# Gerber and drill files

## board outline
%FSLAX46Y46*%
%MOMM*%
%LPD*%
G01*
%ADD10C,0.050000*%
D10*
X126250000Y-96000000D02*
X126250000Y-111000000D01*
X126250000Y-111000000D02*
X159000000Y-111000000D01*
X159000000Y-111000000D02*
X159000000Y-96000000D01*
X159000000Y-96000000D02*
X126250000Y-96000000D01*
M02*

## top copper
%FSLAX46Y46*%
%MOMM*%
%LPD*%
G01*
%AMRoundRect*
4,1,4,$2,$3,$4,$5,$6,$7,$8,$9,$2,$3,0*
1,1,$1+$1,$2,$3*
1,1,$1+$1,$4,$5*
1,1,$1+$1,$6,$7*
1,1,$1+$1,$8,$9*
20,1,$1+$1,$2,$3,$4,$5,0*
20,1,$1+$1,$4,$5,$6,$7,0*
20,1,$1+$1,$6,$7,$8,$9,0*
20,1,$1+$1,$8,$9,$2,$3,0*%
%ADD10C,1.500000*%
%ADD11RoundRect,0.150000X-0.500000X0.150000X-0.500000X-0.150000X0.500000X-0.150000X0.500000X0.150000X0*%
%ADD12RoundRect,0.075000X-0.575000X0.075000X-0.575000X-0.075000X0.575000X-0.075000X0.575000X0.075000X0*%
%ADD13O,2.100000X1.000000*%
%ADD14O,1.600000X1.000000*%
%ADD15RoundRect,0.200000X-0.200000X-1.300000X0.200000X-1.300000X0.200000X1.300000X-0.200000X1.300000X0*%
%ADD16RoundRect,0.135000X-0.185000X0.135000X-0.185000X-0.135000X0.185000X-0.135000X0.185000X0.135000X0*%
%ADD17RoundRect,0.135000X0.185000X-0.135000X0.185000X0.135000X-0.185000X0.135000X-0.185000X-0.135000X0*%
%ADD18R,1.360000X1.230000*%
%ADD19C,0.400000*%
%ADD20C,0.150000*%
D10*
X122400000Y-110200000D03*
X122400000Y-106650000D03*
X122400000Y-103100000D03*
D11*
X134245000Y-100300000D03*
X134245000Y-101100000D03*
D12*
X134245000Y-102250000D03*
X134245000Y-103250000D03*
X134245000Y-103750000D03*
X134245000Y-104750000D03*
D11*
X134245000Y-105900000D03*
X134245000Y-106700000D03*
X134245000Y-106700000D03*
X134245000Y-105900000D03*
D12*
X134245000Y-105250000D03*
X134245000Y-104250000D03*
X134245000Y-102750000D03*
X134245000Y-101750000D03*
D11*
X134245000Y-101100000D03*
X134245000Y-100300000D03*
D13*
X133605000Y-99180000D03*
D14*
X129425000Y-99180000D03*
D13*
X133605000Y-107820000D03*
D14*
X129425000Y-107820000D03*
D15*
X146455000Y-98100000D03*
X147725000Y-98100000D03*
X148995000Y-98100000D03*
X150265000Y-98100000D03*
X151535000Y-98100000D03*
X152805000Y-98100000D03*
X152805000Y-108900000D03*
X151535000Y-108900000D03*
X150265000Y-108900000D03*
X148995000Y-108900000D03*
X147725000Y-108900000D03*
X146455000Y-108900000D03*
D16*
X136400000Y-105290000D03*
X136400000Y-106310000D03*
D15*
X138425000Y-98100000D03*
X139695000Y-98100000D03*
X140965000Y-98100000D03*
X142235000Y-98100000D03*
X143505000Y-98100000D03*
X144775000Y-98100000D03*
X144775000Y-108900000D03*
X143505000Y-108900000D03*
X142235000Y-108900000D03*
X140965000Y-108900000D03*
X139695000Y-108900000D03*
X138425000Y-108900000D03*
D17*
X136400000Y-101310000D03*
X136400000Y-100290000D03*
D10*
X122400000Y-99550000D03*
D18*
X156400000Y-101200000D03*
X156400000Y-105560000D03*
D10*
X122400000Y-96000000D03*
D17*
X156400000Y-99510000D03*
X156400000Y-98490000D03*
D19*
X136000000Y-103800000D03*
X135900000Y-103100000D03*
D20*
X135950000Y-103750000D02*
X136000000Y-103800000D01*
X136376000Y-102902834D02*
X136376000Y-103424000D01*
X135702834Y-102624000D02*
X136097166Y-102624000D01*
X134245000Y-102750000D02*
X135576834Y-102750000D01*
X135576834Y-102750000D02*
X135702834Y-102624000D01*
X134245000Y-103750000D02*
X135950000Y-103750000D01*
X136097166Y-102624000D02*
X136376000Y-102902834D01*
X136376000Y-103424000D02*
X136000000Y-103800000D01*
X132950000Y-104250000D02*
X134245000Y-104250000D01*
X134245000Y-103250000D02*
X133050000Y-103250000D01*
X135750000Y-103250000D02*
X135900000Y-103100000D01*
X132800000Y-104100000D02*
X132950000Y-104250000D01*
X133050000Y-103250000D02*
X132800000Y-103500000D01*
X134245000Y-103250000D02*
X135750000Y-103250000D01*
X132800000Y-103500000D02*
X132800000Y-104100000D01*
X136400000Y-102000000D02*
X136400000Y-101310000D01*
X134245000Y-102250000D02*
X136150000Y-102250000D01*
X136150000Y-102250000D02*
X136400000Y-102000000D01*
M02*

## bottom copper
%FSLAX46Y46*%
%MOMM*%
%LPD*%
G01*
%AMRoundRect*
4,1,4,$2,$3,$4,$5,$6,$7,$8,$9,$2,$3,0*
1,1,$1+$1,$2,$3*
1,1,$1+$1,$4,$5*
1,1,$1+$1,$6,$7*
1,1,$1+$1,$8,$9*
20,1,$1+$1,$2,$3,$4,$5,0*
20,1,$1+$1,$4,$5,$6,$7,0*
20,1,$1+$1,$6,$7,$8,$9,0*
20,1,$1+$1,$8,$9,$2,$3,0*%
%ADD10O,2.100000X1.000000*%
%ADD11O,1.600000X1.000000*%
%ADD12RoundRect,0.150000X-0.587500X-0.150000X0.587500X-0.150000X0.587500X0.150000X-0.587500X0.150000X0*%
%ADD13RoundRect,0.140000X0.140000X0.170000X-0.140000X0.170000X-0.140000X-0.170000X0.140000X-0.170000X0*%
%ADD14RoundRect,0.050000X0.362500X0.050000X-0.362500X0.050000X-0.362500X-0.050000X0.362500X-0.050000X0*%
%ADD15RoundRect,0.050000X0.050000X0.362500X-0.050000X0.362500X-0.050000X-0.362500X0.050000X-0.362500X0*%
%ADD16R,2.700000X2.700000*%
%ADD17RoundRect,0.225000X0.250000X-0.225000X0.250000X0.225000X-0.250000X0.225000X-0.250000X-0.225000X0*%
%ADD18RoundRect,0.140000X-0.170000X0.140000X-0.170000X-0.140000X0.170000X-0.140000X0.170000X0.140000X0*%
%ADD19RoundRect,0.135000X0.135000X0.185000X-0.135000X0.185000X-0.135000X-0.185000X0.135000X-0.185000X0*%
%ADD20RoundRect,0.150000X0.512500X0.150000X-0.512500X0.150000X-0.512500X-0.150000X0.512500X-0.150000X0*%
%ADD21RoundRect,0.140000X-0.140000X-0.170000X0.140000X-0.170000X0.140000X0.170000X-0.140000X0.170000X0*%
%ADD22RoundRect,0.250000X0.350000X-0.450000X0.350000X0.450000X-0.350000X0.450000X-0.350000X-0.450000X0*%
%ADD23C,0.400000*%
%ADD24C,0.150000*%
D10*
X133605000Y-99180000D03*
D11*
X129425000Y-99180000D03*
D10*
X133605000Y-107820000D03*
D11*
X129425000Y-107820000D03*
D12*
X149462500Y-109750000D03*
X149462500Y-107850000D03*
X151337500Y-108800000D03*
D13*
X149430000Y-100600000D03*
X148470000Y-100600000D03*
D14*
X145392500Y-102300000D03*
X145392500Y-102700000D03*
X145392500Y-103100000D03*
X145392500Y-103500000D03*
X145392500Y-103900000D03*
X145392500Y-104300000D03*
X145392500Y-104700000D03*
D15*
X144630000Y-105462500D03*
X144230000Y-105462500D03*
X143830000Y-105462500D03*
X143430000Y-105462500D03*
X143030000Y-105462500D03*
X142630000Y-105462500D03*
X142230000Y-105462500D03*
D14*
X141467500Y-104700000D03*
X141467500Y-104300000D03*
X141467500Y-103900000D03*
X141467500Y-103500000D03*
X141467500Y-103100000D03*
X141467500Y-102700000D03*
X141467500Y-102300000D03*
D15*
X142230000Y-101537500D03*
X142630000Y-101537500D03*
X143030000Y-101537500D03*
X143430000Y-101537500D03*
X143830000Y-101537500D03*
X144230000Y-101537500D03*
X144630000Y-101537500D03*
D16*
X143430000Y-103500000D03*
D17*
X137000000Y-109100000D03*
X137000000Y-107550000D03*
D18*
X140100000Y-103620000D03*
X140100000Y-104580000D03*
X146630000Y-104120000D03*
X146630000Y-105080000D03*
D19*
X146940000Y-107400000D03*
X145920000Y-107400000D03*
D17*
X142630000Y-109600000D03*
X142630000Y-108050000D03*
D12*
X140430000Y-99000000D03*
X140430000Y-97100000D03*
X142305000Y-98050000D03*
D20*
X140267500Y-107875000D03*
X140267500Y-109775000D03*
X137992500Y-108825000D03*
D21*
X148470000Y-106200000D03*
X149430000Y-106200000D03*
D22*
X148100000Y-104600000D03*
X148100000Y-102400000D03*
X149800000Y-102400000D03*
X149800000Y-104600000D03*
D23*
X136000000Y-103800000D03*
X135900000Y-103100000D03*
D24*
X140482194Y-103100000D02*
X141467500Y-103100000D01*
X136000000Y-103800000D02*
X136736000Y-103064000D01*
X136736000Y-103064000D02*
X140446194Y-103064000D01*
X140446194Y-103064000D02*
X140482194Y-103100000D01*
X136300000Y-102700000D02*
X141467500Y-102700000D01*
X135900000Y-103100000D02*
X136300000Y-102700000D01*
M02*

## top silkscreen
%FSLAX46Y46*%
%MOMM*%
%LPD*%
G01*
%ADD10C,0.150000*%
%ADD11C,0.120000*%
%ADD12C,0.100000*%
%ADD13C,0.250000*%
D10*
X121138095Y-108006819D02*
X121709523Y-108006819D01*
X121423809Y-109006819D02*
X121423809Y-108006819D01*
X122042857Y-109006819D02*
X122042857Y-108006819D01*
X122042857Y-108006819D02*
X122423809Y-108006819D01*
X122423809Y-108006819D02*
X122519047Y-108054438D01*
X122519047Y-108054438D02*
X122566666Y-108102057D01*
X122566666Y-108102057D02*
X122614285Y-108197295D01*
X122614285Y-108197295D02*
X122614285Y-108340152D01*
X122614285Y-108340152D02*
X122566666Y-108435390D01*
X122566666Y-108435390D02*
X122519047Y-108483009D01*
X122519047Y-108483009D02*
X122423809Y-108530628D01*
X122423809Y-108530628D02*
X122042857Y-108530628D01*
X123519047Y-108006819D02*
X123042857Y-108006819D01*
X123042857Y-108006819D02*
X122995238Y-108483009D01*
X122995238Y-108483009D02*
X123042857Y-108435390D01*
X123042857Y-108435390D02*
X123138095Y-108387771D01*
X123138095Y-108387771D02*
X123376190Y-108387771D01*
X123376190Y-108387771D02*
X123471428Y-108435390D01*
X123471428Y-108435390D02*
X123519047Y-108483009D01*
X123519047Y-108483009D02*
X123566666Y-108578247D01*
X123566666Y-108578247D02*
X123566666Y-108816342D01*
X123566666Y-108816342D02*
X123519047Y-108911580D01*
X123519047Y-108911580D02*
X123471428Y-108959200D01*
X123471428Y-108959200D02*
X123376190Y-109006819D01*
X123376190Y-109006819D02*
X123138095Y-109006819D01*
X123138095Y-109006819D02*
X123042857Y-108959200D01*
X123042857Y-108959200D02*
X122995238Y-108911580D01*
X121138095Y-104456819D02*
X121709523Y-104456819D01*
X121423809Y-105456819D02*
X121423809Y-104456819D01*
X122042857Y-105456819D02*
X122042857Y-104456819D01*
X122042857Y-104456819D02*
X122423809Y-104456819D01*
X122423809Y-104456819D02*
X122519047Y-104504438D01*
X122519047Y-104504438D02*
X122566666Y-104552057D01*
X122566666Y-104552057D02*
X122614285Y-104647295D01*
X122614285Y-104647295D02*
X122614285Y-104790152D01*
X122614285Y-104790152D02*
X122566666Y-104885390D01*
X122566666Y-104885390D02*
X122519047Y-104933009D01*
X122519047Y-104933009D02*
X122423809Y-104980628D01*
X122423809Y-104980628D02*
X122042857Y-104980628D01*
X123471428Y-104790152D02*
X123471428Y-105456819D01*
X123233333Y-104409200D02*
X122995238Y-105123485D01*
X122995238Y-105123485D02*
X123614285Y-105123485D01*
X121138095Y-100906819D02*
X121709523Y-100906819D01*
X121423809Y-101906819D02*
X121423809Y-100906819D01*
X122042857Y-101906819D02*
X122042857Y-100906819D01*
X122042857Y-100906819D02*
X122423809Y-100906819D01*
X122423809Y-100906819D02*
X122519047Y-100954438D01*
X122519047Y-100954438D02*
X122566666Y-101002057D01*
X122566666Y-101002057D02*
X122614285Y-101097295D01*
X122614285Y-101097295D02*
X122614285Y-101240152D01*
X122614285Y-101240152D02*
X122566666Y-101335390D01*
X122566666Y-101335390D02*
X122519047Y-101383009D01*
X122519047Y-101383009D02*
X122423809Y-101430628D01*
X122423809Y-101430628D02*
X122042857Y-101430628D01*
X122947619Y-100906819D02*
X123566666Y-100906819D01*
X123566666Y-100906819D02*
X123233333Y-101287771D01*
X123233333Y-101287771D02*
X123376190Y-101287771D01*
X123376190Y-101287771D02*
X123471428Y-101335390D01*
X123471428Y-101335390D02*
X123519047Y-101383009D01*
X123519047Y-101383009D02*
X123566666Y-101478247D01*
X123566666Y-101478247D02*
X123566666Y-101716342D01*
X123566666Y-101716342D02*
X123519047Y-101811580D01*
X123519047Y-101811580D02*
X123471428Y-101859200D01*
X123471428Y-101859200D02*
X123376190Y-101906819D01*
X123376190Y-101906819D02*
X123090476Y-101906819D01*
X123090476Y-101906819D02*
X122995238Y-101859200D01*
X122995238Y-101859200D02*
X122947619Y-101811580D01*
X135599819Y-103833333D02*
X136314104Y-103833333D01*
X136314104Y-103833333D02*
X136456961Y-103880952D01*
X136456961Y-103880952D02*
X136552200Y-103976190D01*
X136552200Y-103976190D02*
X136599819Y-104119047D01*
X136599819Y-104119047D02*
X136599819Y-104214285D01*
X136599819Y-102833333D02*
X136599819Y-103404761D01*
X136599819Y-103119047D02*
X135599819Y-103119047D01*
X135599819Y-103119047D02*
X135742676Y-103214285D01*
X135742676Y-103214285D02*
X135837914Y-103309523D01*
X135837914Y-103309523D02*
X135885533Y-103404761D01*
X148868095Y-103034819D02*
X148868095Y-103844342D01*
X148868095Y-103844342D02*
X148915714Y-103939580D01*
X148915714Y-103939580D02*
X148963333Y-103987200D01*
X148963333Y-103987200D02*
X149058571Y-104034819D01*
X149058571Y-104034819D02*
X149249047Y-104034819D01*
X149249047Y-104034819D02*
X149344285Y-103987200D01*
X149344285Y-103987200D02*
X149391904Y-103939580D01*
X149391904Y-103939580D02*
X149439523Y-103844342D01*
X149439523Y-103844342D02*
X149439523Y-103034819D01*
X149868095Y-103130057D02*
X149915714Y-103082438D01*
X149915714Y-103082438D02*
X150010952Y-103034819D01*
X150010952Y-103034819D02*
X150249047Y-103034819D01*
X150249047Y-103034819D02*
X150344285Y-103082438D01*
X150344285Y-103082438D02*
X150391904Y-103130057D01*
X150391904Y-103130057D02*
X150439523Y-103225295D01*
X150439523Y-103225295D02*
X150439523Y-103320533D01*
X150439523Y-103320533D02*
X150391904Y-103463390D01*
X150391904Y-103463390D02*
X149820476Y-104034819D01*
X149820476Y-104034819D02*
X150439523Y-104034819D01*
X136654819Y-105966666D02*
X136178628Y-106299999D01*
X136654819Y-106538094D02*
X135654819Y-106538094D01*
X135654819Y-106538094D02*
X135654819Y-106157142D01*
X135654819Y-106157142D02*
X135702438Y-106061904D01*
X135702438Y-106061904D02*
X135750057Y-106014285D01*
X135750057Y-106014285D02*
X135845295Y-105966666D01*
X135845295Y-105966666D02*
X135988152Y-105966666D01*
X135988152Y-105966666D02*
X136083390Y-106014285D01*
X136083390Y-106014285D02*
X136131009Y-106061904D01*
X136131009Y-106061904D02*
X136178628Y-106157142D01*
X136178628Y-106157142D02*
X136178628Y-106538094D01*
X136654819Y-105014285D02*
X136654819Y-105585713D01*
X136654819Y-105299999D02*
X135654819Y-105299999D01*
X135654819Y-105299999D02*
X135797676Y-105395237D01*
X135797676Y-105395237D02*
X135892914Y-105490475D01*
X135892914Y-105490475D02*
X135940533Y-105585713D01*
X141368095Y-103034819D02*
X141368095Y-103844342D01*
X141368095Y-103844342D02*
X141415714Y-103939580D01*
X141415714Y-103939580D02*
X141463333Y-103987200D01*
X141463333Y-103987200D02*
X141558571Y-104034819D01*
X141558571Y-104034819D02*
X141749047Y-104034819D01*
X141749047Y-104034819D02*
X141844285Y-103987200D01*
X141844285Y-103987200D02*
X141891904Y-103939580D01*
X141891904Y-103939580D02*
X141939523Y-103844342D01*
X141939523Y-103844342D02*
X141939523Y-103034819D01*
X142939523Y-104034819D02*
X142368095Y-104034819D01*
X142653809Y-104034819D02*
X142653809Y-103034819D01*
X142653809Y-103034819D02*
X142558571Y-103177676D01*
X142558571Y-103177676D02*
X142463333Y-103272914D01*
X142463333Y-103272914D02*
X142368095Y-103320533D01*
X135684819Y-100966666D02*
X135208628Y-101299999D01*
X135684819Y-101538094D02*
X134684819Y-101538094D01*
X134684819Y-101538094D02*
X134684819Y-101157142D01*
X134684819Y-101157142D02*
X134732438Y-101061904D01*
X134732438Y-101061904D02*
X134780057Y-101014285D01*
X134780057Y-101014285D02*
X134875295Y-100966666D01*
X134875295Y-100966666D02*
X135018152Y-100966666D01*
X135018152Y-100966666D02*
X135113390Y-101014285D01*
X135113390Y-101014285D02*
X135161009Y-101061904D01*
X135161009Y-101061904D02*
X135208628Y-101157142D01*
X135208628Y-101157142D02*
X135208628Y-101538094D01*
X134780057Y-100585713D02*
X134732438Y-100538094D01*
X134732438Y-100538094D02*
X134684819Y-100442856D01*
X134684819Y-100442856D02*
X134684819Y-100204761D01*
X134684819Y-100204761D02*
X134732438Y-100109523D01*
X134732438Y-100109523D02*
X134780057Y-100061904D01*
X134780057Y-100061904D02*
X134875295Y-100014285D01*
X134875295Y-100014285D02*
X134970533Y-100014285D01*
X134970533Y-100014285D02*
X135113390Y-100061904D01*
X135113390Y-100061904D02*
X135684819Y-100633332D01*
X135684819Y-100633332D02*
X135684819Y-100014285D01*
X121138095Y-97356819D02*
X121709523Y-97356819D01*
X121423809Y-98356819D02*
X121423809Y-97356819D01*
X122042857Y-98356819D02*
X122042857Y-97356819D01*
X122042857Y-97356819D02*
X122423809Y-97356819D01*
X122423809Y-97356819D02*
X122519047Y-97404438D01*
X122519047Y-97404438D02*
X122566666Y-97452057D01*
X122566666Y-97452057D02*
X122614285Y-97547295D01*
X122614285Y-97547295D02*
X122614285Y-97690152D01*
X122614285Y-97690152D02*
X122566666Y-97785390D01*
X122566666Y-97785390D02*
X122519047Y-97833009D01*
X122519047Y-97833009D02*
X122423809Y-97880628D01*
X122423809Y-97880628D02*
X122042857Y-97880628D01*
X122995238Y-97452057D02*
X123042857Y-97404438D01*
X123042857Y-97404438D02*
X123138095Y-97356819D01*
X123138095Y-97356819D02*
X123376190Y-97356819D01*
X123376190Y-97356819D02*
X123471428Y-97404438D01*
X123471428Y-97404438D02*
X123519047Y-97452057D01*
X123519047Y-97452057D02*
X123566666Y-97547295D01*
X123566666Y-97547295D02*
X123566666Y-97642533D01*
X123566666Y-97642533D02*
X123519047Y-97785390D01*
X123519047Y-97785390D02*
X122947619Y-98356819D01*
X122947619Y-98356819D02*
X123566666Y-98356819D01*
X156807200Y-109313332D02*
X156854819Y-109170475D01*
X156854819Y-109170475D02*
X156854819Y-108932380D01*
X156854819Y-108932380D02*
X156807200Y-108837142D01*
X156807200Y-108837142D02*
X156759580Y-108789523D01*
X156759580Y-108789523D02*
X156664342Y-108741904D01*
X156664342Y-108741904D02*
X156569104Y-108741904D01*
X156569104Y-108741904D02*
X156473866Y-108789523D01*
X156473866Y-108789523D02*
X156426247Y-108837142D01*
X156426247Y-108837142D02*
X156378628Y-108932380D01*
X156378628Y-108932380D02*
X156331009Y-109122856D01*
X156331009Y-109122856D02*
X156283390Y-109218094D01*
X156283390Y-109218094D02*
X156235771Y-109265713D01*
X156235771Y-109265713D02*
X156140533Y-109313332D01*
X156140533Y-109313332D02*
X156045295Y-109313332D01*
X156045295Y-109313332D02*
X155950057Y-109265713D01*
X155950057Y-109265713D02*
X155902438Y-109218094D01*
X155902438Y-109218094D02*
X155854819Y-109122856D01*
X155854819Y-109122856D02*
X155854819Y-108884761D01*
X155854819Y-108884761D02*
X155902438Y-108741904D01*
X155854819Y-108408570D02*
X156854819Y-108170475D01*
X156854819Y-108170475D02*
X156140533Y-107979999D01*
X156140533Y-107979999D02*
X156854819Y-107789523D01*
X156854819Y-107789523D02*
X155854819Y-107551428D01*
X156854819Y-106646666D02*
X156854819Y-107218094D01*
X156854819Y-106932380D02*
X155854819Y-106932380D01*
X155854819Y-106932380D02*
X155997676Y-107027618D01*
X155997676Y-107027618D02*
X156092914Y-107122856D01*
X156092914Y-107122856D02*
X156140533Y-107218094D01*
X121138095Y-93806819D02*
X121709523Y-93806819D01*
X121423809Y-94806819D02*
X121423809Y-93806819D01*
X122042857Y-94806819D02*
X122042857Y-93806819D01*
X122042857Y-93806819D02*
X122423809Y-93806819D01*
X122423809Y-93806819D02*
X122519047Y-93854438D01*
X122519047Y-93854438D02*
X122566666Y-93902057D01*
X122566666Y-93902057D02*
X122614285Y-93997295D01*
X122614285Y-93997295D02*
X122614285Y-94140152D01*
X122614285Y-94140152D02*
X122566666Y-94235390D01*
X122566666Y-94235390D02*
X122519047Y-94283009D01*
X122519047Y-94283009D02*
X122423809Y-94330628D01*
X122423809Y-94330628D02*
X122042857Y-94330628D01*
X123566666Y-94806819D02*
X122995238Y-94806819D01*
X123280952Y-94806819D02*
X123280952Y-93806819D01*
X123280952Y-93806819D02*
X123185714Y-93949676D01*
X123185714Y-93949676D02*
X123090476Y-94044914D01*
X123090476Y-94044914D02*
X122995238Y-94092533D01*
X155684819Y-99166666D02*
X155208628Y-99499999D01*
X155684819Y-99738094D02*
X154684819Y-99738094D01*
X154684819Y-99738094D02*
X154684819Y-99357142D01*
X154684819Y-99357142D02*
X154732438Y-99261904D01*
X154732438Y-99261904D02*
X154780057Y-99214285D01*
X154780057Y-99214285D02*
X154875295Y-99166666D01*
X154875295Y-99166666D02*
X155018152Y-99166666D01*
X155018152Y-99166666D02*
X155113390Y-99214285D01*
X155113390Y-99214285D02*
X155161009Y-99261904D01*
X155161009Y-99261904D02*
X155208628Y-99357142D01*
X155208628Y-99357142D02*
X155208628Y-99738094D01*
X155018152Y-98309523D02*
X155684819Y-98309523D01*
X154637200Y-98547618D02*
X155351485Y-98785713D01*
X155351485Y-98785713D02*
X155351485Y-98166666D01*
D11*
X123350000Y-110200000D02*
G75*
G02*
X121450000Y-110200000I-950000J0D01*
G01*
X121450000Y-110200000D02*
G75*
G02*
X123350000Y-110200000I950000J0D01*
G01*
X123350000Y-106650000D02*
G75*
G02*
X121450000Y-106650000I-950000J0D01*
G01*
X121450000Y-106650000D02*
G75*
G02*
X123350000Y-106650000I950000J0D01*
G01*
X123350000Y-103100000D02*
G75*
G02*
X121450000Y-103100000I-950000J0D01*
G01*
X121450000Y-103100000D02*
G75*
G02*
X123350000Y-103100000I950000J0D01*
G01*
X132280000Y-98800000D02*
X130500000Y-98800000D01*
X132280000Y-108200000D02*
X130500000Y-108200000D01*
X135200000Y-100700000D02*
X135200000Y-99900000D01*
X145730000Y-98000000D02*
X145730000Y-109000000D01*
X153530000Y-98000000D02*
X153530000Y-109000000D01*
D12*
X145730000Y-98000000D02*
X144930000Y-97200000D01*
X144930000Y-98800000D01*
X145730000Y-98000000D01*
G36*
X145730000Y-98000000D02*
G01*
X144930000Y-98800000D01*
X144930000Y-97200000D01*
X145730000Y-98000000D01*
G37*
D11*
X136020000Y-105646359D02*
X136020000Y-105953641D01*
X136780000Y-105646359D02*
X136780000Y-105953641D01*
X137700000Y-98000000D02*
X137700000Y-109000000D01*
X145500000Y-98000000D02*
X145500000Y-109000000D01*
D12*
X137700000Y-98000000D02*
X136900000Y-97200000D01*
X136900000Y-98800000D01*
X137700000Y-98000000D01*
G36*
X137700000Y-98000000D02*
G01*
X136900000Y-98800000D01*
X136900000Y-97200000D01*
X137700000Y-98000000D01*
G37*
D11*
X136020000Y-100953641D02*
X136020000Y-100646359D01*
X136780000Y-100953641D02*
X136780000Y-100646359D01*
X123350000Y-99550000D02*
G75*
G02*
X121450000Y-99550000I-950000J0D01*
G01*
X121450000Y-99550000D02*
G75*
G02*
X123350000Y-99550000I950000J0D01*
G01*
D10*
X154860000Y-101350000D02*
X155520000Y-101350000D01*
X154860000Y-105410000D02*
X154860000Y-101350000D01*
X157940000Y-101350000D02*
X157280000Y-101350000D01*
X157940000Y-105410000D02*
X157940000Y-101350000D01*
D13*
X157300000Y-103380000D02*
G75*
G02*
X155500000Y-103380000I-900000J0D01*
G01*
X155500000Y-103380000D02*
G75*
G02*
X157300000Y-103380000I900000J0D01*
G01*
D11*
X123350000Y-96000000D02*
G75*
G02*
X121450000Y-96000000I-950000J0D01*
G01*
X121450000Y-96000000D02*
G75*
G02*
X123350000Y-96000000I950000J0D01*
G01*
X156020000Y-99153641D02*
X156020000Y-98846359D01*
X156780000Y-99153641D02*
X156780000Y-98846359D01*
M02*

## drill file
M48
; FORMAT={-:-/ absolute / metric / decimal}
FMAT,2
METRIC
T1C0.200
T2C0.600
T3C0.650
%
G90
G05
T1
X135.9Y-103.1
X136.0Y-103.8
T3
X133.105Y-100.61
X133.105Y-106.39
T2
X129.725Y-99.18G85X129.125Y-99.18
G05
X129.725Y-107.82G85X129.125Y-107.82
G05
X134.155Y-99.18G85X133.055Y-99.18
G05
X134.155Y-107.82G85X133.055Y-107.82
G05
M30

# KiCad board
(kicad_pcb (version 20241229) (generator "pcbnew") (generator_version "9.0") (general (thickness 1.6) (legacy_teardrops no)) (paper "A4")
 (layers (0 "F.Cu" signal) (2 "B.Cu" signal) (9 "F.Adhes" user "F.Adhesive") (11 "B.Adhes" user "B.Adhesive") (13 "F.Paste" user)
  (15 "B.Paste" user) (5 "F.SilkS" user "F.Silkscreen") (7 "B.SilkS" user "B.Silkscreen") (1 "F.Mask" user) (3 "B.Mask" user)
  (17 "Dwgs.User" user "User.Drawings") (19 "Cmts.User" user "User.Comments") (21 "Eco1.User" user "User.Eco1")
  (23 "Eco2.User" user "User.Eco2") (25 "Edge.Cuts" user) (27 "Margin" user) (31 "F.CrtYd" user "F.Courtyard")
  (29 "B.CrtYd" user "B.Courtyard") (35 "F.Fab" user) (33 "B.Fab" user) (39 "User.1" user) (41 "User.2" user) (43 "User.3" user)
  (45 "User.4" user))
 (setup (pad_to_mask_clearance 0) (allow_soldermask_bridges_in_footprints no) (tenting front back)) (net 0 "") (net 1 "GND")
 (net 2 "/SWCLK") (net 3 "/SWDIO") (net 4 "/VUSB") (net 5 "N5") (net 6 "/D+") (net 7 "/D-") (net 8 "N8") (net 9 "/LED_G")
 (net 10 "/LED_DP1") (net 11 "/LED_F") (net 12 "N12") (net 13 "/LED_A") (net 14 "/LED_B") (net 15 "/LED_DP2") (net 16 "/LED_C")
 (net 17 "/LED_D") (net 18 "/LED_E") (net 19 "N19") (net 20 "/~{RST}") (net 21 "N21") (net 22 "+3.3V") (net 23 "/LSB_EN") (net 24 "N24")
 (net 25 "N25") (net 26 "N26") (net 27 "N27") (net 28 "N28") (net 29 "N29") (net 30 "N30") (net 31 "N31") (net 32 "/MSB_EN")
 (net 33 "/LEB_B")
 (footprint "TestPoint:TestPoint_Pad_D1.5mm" (layer "F.Cu") (at 122.4 110.2)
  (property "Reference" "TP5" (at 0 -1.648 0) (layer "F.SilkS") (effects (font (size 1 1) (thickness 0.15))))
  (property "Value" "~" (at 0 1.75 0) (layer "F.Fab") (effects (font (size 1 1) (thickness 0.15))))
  (fp_circle (center 0 0) (end 0 0.95) (stroke (width 0.12) (type solid)) (fill no) (layer "F.SilkS"))
  (pad "1" smd circle (at 0 0) (size 1.5 1.5) (layers "F.Cu" "F.Mask") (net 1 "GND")))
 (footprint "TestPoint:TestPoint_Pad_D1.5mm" (layer "F.Cu") (at 122.4 106.65)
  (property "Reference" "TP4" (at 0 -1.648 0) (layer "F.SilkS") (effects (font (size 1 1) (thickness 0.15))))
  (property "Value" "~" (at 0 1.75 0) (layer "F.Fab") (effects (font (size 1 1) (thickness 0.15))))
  (fp_circle (center 0 0) (end 0 0.95) (stroke (width 0.12) (type solid)) (fill no) (layer "F.SilkS"))
  (pad "1" smd circle (at 0 0) (size 1.5 1.5) (layers "F.Cu" "F.Mask") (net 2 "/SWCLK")))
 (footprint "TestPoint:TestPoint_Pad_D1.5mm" (layer "F.Cu") (at 122.4 103.1)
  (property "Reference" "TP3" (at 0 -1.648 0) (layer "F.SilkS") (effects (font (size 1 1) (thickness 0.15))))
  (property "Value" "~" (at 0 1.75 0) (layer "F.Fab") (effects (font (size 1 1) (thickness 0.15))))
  (fp_circle (center 0 0) (end 0 0.95) (stroke (width 0.12) (type solid)) (fill no) (layer "F.SilkS"))
  (pad "1" smd circle (at 0 0) (size 1.5 1.5) (layers "F.Cu" "F.Mask") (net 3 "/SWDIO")))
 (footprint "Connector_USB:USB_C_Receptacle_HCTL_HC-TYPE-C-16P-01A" (layer "F.Cu") (at 130.5 103.5 -90)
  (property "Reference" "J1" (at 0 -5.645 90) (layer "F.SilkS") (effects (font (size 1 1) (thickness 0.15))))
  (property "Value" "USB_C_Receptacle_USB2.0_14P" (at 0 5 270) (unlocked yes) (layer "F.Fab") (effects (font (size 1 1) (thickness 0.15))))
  (fp_line (start -4.7 -1.78) (end -4.7 0) (stroke (width 0.12) (type solid)) (layer "F.SilkS"))
  (fp_line (start 4.7 -1.78) (end 4.7 0) (stroke (width 0.12) (type solid)) (layer "F.SilkS"))
  (fp_line (start -2.8 -4.7) (end -3.6 -4.7) (stroke (width 0.12) (type default)) (layer "F.SilkS"))
  (pad "" np_thru_hole circle (at -2.89 -2.605 270) (size 0.65 0.65) (drill 0.65) (layers "*.Mask"))
  (pad "" np_thru_hole circle (at 2.89 -2.605 270) (size 0.65 0.65) (drill 0.65) (layers "*.Mask"))
  (pad "A1" smd roundrect (at -3.2 -3.745 270) (size 0.6 1.3) (layers "F.Cu" "F.Mask" "F.Paste") (roundrect_rratio 0.25) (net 1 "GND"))
  (pad "A4" smd roundrect (at -2.4 -3.745 270) (size 0.6 1.3) (layers "F.Cu" "F.Mask" "F.Paste") (roundrect_rratio 0.25) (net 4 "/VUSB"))
  (pad "A5" smd roundrect (at -1.25 -3.745 270) (size 0.3 1.3) (layers "F.Cu" "F.Mask" "F.Paste") (roundrect_rratio 0.25) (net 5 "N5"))
  (pad "A6" smd roundrect (at -0.25 -3.745 270) (size 0.3 1.3) (layers "F.Cu" "F.Mask" "F.Paste") (roundrect_rratio 0.25) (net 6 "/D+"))
  (pad "A7" smd roundrect (at 0.25 -3.745 270) (size 0.3 1.3) (layers "F.Cu" "F.Mask" "F.Paste") (roundrect_rratio 0.25) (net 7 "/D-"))
  (pad "A8" smd roundrect (at 1.25 -3.745 270) (size 0.3 1.3) (layers "F.Cu" "F.Mask" "F.Paste") (roundrect_rratio 0.25))
  (pad "A9" smd roundrect (at 2.4 -3.745 270) (size 0.6 1.3) (layers "F.Cu" "F.Mask" "F.Paste") (roundrect_rratio 0.25) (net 4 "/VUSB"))
  (pad "A12" smd roundrect (at 3.2 -3.745 270) (size 0.6 1.3) (layers "F.Cu" "F.Mask" "F.Paste") (roundrect_rratio 0.25) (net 1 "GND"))
  (pad "B1" smd roundrect (at 3.2 -3.745 270) (size 0.6 1.3) (layers "F.Cu" "F.Mask" "F.Paste") (roundrect_rratio 0.25) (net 1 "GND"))
  (pad "B4" smd roundrect (at 2.4 -3.745 270) (size 0.6 1.3) (layers "F.Cu" "F.Mask" "F.Paste") (roundrect_rratio 0.25) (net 4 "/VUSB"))
  (pad "B5" smd roundrect (at 1.75 -3.745 270) (size 0.3 1.3) (layers "F.Cu" "F.Mask" "F.Paste") (roundrect_rratio 0.25) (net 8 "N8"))
  (pad "B6" smd roundrect (at 0.75 -3.745 270) (size 0.3 1.3) (layers "F.Cu" "F.Mask" "F.Paste") (roundrect_rratio 0.25) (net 6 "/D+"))
  (pad "B7" smd roundrect (at -0.75 -3.745 270) (size 0.3 1.3) (layers "F.Cu" "F.Mask" "F.Paste") (roundrect_rratio 0.25) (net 7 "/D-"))
  (pad "B8" smd roundrect (at -1.75 -3.745 270) (size 0.3 1.3) (layers "F.Cu" "F.Mask" "F.Paste") (roundrect_rratio 0.25))
  (pad "B9" smd roundrect (at -2.4 -3.745 270) (size 0.6 1.3) (layers "F.Cu" "F.Mask" "F.Paste") (roundrect_rratio 0.25) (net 4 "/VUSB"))
  (pad "B12" smd roundrect (at -3.2 -3.745 270) (size 0.6 1.3) (layers "F.Cu" "F.Mask" "F.Paste") (roundrect_rratio 0.25) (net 1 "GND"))
  (pad "S1" thru_hole oval (at -4.32 -3.105 270) (size 1 2.1) (drill oval 0.6 1.7) (layers "*.Cu" "*.Mask") (remove_unused_layers no)
   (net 1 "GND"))
  (pad "S1" thru_hole oval (at -4.32 1.075 270) (size 1 1.6) (drill oval 0.6 1.2) (layers "*.Cu" "*.Mask") (remove_unused_layers no)
   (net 1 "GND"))
  (pad "S1" thru_hole oval (at 4.32 -3.105 270) (size 1 2.1) (drill oval 0.6 1.7) (layers "*.Cu" "*.Mask") (remove_unused_layers no)
   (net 1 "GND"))
  (pad "S1" thru_hole oval (at 4.32 1.075 270) (size 1 1.6) (drill oval 0.6 1.2) (layers "*.Cu" "*.Mask") (remove_unused_layers no)
   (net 1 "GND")))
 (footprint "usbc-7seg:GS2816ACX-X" (layer "F.Cu") (at 149.63 103.5)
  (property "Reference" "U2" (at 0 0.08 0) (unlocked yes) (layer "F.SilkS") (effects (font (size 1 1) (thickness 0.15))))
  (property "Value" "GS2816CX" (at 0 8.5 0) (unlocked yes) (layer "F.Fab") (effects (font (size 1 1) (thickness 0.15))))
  (fp_line (start -3.9 -5.5) (end -3.9 5.5) (stroke (width 0.12) (type solid)) (layer "F.SilkS"))
  (fp_line (start 3.9 -5.5) (end 3.9 5.5) (stroke (width 0.12) (type solid)) (layer "F.SilkS"))
  (fp_poly (pts (xy -3.9 -5.5) (xy -4.7 -6.3) (xy -4.7 -4.7)) (stroke (width 0.1) (type solid)) (fill yes) (layer "F.SilkS"))
  (pad "1" smd roundrect (at -3.175 -5.4) (size 0.8 3) (layers "F.Cu" "F.Mask" "F.Paste") (roundrect_rratio 0.25) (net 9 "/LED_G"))
  (pad "2" smd roundrect (at -1.905 -5.4) (size 0.8 3) (layers "F.Cu" "F.Mask" "F.Paste") (roundrect_rratio 0.25) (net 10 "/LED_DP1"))
  (pad "3" smd roundrect (at -0.635 -5.4) (size 0.8 3) (layers "F.Cu" "F.Mask" "F.Paste") (roundrect_rratio 0.25) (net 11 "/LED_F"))
  (pad "4" smd roundrect (at 0.635 -5.4) (size 0.8 3) (layers "F.Cu" "F.Mask" "F.Paste") (roundrect_rratio 0.25) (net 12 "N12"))
  (pad "5" smd roundrect (at 1.905 -5.4) (size 0.8 3) (layers "F.Cu" "F.Mask" "F.Paste") (roundrect_rratio 0.25) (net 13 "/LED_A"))
  (pad "6" smd roundrect (at 3.175 -5.4) (size 0.8 3) (layers "F.Cu" "F.Mask" "F.Paste") (roundrect_rratio 0.25) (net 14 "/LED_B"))
  (pad "7" smd roundrect (at 3.175 5.4) (size 0.8 3) (layers "F.Cu" "F.Mask" "F.Paste") (roundrect_rratio 0.25) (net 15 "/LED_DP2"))
  (pad "8" smd roundrect (at 1.905 5.4) (size 0.8 3) (layers "F.Cu" "F.Mask" "F.Paste") (roundrect_rratio 0.25) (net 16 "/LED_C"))
  (pad "9" smd roundrect (at 0.635 5.4) (size 0.8 3) (layers "F.Cu" "F.Mask" "F.Paste") (roundrect_rratio 0.25) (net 12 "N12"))
  (pad "10" smd roundrect (at -0.635 5.4) (size 0.8 3) (layers "F.Cu" "F.Mask" "F.Paste") (roundrect_rratio 0.25) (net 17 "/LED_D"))
  (pad "11" smd roundrect (at -1.905 5.4) (size 0.8 3) (layers "F.Cu" "F.Mask" "F.Paste") (roundrect_rratio 0.25) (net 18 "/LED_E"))
  (pad "12" smd roundrect (at -3.175 5.4) (size 0.8 3) (layers "F.Cu" "F.Mask" "F.Paste") (roundrect_rratio 0.25)))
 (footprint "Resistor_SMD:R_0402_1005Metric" (layer "F.Cu") (at 136.4 105.8 -90)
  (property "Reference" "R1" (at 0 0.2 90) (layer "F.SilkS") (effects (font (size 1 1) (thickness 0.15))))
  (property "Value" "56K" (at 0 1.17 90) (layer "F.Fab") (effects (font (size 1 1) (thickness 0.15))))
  (fp_line (start -0.153641 0.38) (end 0.153641 0.38) (stroke (width 0.12) (type solid)) (layer "F.SilkS"))
  (fp_line (start -0.153641 -0.38) (end 0.153641 -0.38) (stroke (width 0.12) (type solid)) (layer "F.SilkS"))
  (pad "1" smd roundrect (at -0.51 0 270) (size 0.54 0.64) (layers "F.Cu" "F.Mask" "F.Paste") (roundrect_rratio 0.25) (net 8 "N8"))
  (pad "2" smd roundrect (at 0.51 0 270) (size 0.54 0.64) (layers "F.Cu" "F.Mask" "F.Paste") (roundrect_rratio 0.25) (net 1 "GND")))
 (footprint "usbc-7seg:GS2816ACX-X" (layer "F.Cu") (at 141.6 103.5)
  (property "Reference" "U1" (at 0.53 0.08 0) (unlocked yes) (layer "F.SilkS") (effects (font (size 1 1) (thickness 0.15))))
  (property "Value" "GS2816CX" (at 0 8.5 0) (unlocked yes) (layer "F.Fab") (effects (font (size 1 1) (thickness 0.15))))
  (fp_line (start -3.9 -5.5) (end -3.9 5.5) (stroke (width 0.12) (type solid)) (layer "F.SilkS"))
  (fp_line (start 3.9 -5.5) (end 3.9 5.5) (stroke (width 0.12) (type solid)) (layer "F.SilkS"))
  (fp_poly (pts (xy -3.9 -5.5) (xy -4.7 -6.3) (xy -4.7 -4.7)) (stroke (width 0.1) (type solid)) (fill yes) (layer "F.SilkS"))
  (pad "1" smd roundrect (at -3.175 -5.4) (size 0.8 3) (layers "F.Cu" "F.Mask" "F.Paste") (roundrect_rratio 0.25) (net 9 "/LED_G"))
  (pad "2" smd roundrect (at -1.905 -5.4) (size 0.8 3) (layers "F.Cu" "F.Mask" "F.Paste") (roundrect_rratio 0.25) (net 10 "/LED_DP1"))
  (pad "3" smd roundrect (at -0.635 -5.4) (size 0.8 3) (layers "F.Cu" "F.Mask" "F.Paste") (roundrect_rratio 0.25) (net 11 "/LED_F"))
  (pad "4" smd roundrect (at 0.635 -5.4) (size 0.8 3) (layers "F.Cu" "F.Mask" "F.Paste") (roundrect_rratio 0.25) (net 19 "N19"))
  (pad "5" smd roundrect (at 1.905 -5.4) (size 0.8 3) (layers "F.Cu" "F.Mask" "F.Paste") (roundrect_rratio 0.25) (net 13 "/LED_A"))
  (pad "6" smd roundrect (at 3.175 -5.4) (size 0.8 3) (layers "F.Cu" "F.Mask" "F.Paste") (roundrect_rratio 0.25) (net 14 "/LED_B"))
  (pad "7" smd roundrect (at 3.175 5.4) (size 0.8 3) (layers "F.Cu" "F.Mask" "F.Paste") (roundrect_rratio 0.25) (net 15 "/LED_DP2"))
  (pad "8" smd roundrect (at 1.905 5.4) (size 0.8 3) (layers "F.Cu" "F.Mask" "F.Paste") (roundrect_rratio 0.25) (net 16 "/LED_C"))
  (pad "9" smd roundrect (at 0.635 5.4) (size 0.8 3) (layers "F.Cu" "F.Mask" "F.Paste") (roundrect_rratio 0.25) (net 19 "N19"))
  (pad "10" smd roundrect (at -0.635 5.4) (size 0.8 3) (layers "F.Cu" "F.Mask" "F.Paste") (roundrect_rratio 0.25) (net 17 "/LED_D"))
  (pad "11" smd roundrect (at -1.905 5.4) (size 0.8 3) (layers "F.Cu" "F.Mask" "F.Paste") (roundrect_rratio 0.25) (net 18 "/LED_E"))
  (pad "12" smd roundrect (at -3.175 5.4) (size 0.8 3) (layers "F.Cu" "F.Mask" "F.Paste") (roundrect_rratio 0.25)))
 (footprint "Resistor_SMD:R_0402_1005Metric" (layer "F.Cu") (at 136.4 100.8 90)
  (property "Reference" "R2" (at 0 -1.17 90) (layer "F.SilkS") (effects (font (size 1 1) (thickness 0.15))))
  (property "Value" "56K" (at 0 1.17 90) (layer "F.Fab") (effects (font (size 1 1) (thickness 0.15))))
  (fp_line (start -0.153641 -0.38) (end 0.153641 -0.38) (stroke (width 0.12) (type solid)) (layer "F.SilkS"))
  (fp_line (start -0.153641 0.38) (end 0.153641 0.38) (stroke (width 0.12) (type solid)) (layer "F.SilkS"))
  (pad "1" smd roundrect (at -0.51 0 90) (size 0.54 0.64) (layers "F.Cu" "F.Mask" "F.Paste") (roundrect_rratio 0.25) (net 5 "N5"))
  (pad "2" smd roundrect (at 0.51 0 90) (size 0.54 0.64) (layers "F.Cu" "F.Mask" "F.Paste") (roundrect_rratio 0.25) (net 1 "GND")))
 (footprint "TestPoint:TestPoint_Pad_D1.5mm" (layer "F.Cu") (at 122.4 99.55)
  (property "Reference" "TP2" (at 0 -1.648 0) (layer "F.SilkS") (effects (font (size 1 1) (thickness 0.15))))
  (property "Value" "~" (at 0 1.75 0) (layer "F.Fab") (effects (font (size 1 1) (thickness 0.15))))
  (fp_circle (center 0 0) (end 0 0.95) (stroke (width 0.12) (type solid)) (fill no) (layer "F.SilkS"))
  (pad "1" smd circle (at 0 0) (size 1.5 1.5) (layers "F.Cu" "F.Mask") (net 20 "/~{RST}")))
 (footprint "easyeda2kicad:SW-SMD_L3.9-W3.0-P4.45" (layer "F.Cu") (at 156.4 103.38 -90)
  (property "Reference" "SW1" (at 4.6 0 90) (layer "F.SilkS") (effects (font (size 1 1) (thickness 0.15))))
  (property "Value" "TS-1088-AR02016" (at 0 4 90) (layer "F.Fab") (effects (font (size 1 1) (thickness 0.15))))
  (fp_line (start -2.03 1.54) (end -2.03 0.88) (stroke (width 0.15) (type solid)) (layer "F.SilkS"))
  (fp_line (start 2.03 1.54) (end -2.03 1.54) (stroke (width 0.15) (type solid)) (layer "F.SilkS"))
  (fp_line (start -2.03 -1.54) (end -2.03 -0.88) (stroke (width 0.15) (type solid)) (layer "F.SilkS"))
  (fp_line (start 2.03 -1.54) (end -2.03 -1.54) (stroke (width 0.15) (type solid)) (layer "F.SilkS"))
  (fp_circle (center 0 0) (end 0.9 0) (stroke (width 0.25) (type solid)) (fill no) (layer "F.SilkS"))
  (pad "1" smd rect (at -2.18 0 270) (size 1.23 1.36) (layers "F.Cu" "F.Mask" "F.Paste") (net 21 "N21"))
  (pad "2" smd rect (at 2.18 0 270) (size 1.23 1.36) (layers "F.Cu" "F.Mask" "F.Paste") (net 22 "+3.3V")))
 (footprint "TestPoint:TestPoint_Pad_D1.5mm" (layer "F.Cu") (at 122.4 96)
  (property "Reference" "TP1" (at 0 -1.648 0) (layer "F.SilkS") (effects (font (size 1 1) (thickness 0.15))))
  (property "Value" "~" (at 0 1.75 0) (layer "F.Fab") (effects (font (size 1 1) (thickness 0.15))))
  (fp_circle (center 0 0) (end 0 0.95) (stroke (width 0.12) (type solid)) (fill no) (layer "F.SilkS"))
  (pad "1" smd circle (at 0 0) (size 1.5 1.5) (layers "F.Cu" "F.Mask") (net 22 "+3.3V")))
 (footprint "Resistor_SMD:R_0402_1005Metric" (layer "F.Cu") (at 156.4 99 90)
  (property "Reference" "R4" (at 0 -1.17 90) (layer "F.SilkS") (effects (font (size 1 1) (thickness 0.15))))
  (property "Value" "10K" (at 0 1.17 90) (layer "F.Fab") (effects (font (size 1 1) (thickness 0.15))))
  (fp_line (start -0.153641 -0.38) (end 0.153641 -0.38) (stroke (width 0.12) (type solid)) (layer "F.SilkS"))
  (fp_line (start -0.153641 0.38) (end 0.153641 0.38) (stroke (width 0.12) (type solid)) (layer "F.SilkS"))
  (pad "1" smd roundrect (at -0.51 0 90) (size 0.54 0.64) (layers "F.Cu" "F.Mask" "F.Paste") (roundrect_rratio 0.25) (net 21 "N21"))
  (pad "2" smd roundrect (at 0.51 0 90) (size 0.54 0.64) (layers "F.Cu" "F.Mask" "F.Paste") (roundrect_rratio 0.25) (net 1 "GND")))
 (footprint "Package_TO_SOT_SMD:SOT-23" (layer "B.Cu") (at 150.4 108.8)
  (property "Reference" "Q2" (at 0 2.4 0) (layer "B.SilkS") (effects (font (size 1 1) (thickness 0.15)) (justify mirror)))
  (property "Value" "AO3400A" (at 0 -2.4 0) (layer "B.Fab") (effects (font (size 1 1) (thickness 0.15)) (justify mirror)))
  (pad "1" smd roundrect (at -0.9375 0.95) (size 1.475 0.6) (layers "B.Cu" "B.Mask" "B.Paste") (roundrect_rratio 0.25) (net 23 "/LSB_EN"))
  (pad "2" smd roundrect (at -0.9375 -0.95) (size 1.475 0.6) (layers "B.Cu" "B.Mask" "B.Paste") (roundrect_rratio 0.25) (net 1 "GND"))
  (pad "3" smd roundrect (at 0.9375 0) (size 1.475 0.6) (layers "B.Cu" "B.Mask" "B.Paste") (roundrect_rratio 0.25) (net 12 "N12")))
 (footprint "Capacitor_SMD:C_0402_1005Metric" (layer "B.Cu") (at 148.95 100.6 180)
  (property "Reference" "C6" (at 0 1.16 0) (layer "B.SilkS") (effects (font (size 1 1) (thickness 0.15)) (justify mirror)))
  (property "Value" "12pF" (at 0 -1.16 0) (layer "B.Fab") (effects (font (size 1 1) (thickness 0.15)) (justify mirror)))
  (pad "1" smd roundrect (at -0.48 0 180) (size 0.56 0.62) (layers "B.Cu" "B.Mask" "B.Paste") (roundrect_rratio 0.25) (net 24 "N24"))
  (pad "2" smd roundrect (at 0.48 0 180) (size 0.56 0.62) (layers "B.Cu" "B.Mask" "B.Paste") (roundrect_rratio 0.25) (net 1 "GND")))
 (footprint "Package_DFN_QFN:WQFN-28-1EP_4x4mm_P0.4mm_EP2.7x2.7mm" (layer "B.Cu") (at 143.43 103.5 180)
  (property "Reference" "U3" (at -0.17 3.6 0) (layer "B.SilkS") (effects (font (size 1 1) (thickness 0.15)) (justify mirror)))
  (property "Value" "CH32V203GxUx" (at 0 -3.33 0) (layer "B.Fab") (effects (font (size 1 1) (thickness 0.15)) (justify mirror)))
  (pad "" smd roundrect (at -0.675 -0.675 180) (size 1.09 1.09) (layers "B.Paste") (roundrect_rratio 0.229358))
  (pad "" smd roundrect (at -0.675 0.675 180) (size 1.09 1.09) (layers "B.Paste") (roundrect_rratio 0.229358))
  (pad "" smd roundrect (at 0.675 -0.675 180) (size 1.09 1.09) (layers "B.Paste") (roundrect_rratio 0.229358))
  (pad "" smd roundrect (at 0.675 0.675 180) (size 1.09 1.09) (layers "B.Paste") (roundrect_rratio 0.229358))
  (pad "1" smd roundrect (at -1.9625 1.2 180) (size 0.825 0.2) (layers "B.Cu" "B.Mask" "B.Paste") (roundrect_rratio 0.25) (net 21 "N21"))
  (pad "2" smd roundrect (at -1.9625 0.8 180) (size 0.825 0.2) (layers "B.Cu" "B.Mask" "B.Paste") (roundrect_rratio 0.25) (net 24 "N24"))
  (pad "3" smd roundrect (at -1.9625 0.4 180) (size 0.825 0.2) (layers "B.Cu" "B.Mask" "B.Paste") (roundrect_rratio 0.25) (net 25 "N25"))
  (pad "4" smd roundrect (at -1.9625 0 180) (size 0.825 0.2) (layers "B.Cu" "B.Mask" "B.Paste") (roundrect_rratio 0.25) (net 20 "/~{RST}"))
  (pad "5" smd roundrect (at -1.9625 -0.4 180) (size 0.825 0.2) (layers "B.Cu" "B.Mask" "B.Paste") (roundrect_rratio 0.25) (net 22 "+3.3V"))
  (pad "6" smd roundrect (at -1.9625 -0.8 180) (size 0.825 0.2) (layers "B.Cu" "B.Mask" "B.Paste") (roundrect_rratio 0.25) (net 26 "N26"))
  (pad "7" smd roundrect (at -1.9625 -1.2 180) (size 0.825 0.2) (layers "B.Cu" "B.Mask" "B.Paste") (roundrect_rratio 0.25)
   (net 23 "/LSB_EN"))
  (pad "8" smd roundrect (at -1.2 -1.9625 180) (size 0.2 0.825) (layers "B.Cu" "B.Mask" "B.Paste") (roundrect_rratio 0.25) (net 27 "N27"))
  (pad "9" smd roundrect (at -0.8 -1.9625 180) (size 0.2 0.825) (layers "B.Cu" "B.Mask" "B.Paste") (roundrect_rratio 0.25) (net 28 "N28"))
  (pad "10" smd roundrect (at -0.4 -1.9625 180) (size 0.2 0.825) (layers "B.Cu" "B.Mask" "B.Paste") (roundrect_rratio 0.25) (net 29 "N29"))
  (pad "11" smd roundrect (at 0 -1.9625 180) (size 0.2 0.825) (layers "B.Cu" "B.Mask" "B.Paste") (roundrect_rratio 0.25) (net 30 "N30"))
  (pad "12" smd roundrect (at 0.4 -1.9625 180) (size 0.2 0.825) (layers "B.Cu" "B.Mask" "B.Paste") (roundrect_rratio 0.25)
   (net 15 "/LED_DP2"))
  (pad "13" smd roundrect (at 0.8 -1.9625 180) (size 0.2 0.825) (layers "B.Cu" "B.Mask" "B.Paste") (roundrect_rratio 0.25) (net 16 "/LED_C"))
  (pad "14" smd roundrect (at 1.2 -1.9625 180) (size 0.2 0.825) (layers "B.Cu" "B.Mask" "B.Paste") (roundrect_rratio 0.25) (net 17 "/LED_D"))
  (pad "15" smd roundrect (at 1.9625 -1.2 180) (size 0.825 0.2) (layers "B.Cu" "B.Mask" "B.Paste") (roundrect_rratio 0.25) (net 18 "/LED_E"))
  (pad "16" smd roundrect (at 1.9625 -0.8 180) (size 0.825 0.2) (layers "B.Cu" "B.Mask" "B.Paste") (roundrect_rratio 0.25) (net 1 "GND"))
  (pad "17" smd roundrect (at 1.9625 -0.4 180) (size 0.825 0.2) (layers "B.Cu" "B.Mask" "B.Paste") (roundrect_rratio 0.25) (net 22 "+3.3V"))
  (pad "18" smd roundrect (at 1.9625 0 180) (size 0.825 0.2) (layers "B.Cu" "B.Mask" "B.Paste") (roundrect_rratio 0.25) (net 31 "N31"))
  (pad "19" smd roundrect (at 1.9625 0.4 180) (size 0.825 0.2) (layers "B.Cu" "B.Mask" "B.Paste") (roundrect_rratio 0.25) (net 7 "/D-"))
  (pad "20" smd roundrect (at 1.9625 0.8 180) (size 0.825 0.2) (layers "B.Cu" "B.Mask" "B.Paste") (roundrect_rratio 0.25) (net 6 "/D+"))
  (pad "21" smd roundrect (at 1.9625 1.2 180) (size 0.825 0.2) (layers "B.Cu" "B.Mask" "B.Paste") (roundrect_rratio 0.25) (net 3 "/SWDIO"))
  (pad "22" smd roundrect (at 1.2 1.9625 180) (size 0.2 0.825) (layers "B.Cu" "B.Mask" "B.Paste") (roundrect_rratio 0.25) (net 2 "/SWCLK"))
  (pad "23" smd roundrect (at 0.8 1.9625 180) (size 0.2 0.825) (layers "B.Cu" "B.Mask" "B.Paste") (roundrect_rratio 0.25) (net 9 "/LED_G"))
  (pad "24" smd roundrect (at 0.4 1.9625 180) (size 0.2 0.825) (layers "B.Cu" "B.Mask" "B.Paste") (roundrect_rratio 0.25)
   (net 10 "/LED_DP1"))
  (pad "25" smd roundrect (at 0 1.9625 180) (size 0.2 0.825) (layers "B.Cu" "B.Mask" "B.Paste") (roundrect_rratio 0.25) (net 11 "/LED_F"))
  (pad "26" smd roundrect (at -0.4 1.9625 180) (size 0.2 0.825) (layers "B.Cu" "B.Mask" "B.Paste") (roundrect_rratio 0.25)
   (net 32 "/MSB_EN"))
  (pad "27" smd roundrect (at -0.8 1.9625 180) (size 0.2 0.825) (layers "B.Cu" "B.Mask" "B.Paste") (roundrect_rratio 0.25) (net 13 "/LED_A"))
  (pad "28" smd roundrect (at -1.2 1.9625 180) (size 0.2 0.825) (layers "B.Cu" "B.Mask" "B.Paste") (roundrect_rratio 0.25) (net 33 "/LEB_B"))
  (pad "29" smd rect (at 0 0 180) (size 2.7 2.7) (layers "B.Cu" "B.Mask") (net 1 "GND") (zone_connect 2)))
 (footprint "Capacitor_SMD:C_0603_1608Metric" (layer "B.Cu") (at 137 108.325 90)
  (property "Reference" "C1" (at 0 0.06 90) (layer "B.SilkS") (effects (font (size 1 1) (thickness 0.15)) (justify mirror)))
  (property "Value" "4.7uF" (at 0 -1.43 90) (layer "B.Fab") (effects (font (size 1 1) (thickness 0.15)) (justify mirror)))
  (pad "1" smd roundrect (at -0.775 0 90) (size 0.9 0.95) (layers "B.Cu" "B.Mask" "B.Paste") (roundrect_rratio 0.25) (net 4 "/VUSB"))
  (pad "2" smd roundrect (at 0.775 0 90) (size 0.9 0.95) (layers "B.Cu" "B.Mask" "B.Paste") (roundrect_rratio 0.25) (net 1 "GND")))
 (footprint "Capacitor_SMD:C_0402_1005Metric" (layer "B.Cu") (at 140.1 104.1 -90)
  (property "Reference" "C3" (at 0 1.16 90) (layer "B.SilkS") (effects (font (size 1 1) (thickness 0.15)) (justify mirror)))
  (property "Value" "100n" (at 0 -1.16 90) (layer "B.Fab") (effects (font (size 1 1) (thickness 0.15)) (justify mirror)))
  (pad "1" smd roundrect (at -0.48 0 270) (size 0.56 0.62) (layers "B.Cu" "B.Mask" "B.Paste") (roundrect_rratio 0.25) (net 22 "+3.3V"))
  (pad "2" smd roundrect (at 0.48 0 270) (size 0.56 0.62) (layers "B.Cu" "B.Mask" "B.Paste") (roundrect_rratio 0.25) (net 1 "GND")))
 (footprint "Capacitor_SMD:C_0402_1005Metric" (layer "B.Cu") (at 146.63 104.6 -90)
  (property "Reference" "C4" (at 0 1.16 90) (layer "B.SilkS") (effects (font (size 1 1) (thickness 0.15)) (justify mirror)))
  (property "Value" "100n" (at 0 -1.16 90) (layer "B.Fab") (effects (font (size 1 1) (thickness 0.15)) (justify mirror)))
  (pad "1" smd roundrect (at -0.48 0 270) (size 0.56 0.62) (layers "B.Cu" "B.Mask" "B.Paste") (roundrect_rratio 0.25) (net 22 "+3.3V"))
  (pad "2" smd roundrect (at 0.48 0 270) (size 0.56 0.62) (layers "B.Cu" "B.Mask" "B.Paste") (roundrect_rratio 0.25) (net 1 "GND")))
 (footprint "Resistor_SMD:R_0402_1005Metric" (layer "B.Cu") (at 146.43 107.4 180)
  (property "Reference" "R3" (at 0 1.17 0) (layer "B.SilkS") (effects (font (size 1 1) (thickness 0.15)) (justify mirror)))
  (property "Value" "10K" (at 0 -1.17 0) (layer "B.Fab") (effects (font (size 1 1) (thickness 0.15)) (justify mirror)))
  (pad "1" smd roundrect (at -0.51 0 180) (size 0.54 0.64) (layers "B.Cu" "B.Mask" "B.Paste") (roundrect_rratio 0.25) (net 22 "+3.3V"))
  (pad "2" smd roundrect (at 0.51 0 180) (size 0.54 0.64) (layers "B.Cu" "B.Mask" "B.Paste") (roundrect_rratio 0.25) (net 20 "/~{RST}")))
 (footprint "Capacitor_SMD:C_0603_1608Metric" (layer "B.Cu") (at 142.63 108.825 90)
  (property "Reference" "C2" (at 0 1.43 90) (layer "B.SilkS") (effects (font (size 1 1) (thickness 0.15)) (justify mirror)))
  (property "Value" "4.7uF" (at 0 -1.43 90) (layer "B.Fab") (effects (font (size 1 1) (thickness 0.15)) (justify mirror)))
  (pad "1" smd roundrect (at -0.775 0 90) (size 0.9 0.95) (layers "B.Cu" "B.Mask" "B.Paste") (roundrect_rratio 0.25) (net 22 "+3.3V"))
  (pad "2" smd roundrect (at 0.775 0 90) (size 0.9 0.95) (layers "B.Cu" "B.Mask" "B.Paste") (roundrect_rratio 0.25) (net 1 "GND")))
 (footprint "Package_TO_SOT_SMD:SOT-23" (layer "B.Cu") (at 141.3675 98.05)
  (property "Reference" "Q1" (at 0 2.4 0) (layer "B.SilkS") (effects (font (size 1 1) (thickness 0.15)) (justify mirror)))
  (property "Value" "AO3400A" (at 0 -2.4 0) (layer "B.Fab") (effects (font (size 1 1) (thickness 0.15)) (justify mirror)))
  (pad "1" smd roundrect (at -0.9375 0.95) (size 1.475 0.6) (layers "B.Cu" "B.Mask" "B.Paste") (roundrect_rratio 0.25) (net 32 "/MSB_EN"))
  (pad "2" smd roundrect (at -0.9375 -0.95) (size 1.475 0.6) (layers "B.Cu" "B.Mask" "B.Paste") (roundrect_rratio 0.25) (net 1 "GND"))
  (pad "3" smd roundrect (at 0.9375 0) (size 1.475 0.6) (layers "B.Cu" "B.Mask" "B.Paste") (roundrect_rratio 0.25) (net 19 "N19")))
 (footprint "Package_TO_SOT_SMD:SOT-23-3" (layer "B.Cu") (at 139.13 108.825 180)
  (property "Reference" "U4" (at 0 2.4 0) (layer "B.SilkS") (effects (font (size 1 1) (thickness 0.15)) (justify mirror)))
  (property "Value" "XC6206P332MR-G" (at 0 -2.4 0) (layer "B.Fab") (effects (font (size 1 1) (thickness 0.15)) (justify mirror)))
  (pad "1" smd roundrect (at -1.1375 0.95 180) (size 1.325 0.6) (layers "B.Cu" "B.Mask" "B.Paste") (roundrect_rratio 0.25) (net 1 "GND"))
  (pad "2" smd roundrect (at -1.1375 -0.95 180) (size 1.325 0.6) (layers "B.Cu" "B.Mask" "B.Paste") (roundrect_rratio 0.25) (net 22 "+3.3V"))
  (pad "3" smd roundrect (at 1.1375 0 180) (size 1.325 0.6) (layers "B.Cu" "B.Mask" "B.Paste") (roundrect_rratio 0.25) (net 4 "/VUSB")))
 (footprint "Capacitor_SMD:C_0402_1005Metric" (layer "B.Cu") (at 148.95 106.2)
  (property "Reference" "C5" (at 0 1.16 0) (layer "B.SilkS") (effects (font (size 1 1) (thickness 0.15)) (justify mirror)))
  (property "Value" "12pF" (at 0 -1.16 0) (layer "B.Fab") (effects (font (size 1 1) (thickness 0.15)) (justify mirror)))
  (pad "1" smd roundrect (at -0.48 0) (size 0.56 0.62) (layers "B.Cu" "B.Mask" "B.Paste") (roundrect_rratio 0.25) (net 25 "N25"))
  (pad "2" smd roundrect (at 0.48 0) (size 0.56 0.62) (layers "B.Cu" "B.Mask" "B.Paste") (roundrect_rratio 0.25) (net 1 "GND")))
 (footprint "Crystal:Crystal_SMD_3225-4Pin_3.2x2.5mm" (layer "B.Cu") (at 148.95 103.5 90)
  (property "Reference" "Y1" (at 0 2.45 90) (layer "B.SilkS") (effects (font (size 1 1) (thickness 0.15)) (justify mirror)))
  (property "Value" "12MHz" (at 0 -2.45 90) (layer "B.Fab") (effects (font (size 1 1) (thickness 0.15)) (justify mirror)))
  (pad "1" smd roundrect (at -1.1 -0.85 90) (size 1.4 1.2) (layers "B.Cu" "B.Mask" "B.Paste") (roundrect_rratio 0.208333) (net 25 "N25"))
  (pad "2" smd roundrect (at 1.1 -0.85 90) (size 1.4 1.2) (layers "B.Cu" "B.Mask" "B.Paste") (roundrect_rratio 0.208333) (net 1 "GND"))
  (pad "3" smd roundrect (at 1.1 0.85 90) (size 1.4 1.2) (layers "B.Cu" "B.Mask" "B.Paste") (roundrect_rratio 0.208333) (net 24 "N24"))
  (pad "4" smd roundrect (at -1.1 0.85 90) (size 1.4 1.2) (layers "B.Cu" "B.Mask" "B.Paste") (roundrect_rratio 0.208333) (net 1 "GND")))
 (gr_line (start 126.25 96) (end 126.25 111) (stroke (width 0.05) (type default)) (layer "Edge.Cuts"))
 (gr_line (start 126.25 111) (end 159 111) (stroke (width 0.05) (type default)) (layer "Edge.Cuts"))
 (gr_line (start 159 111) (end 159 96) (stroke (width 0.05) (type default)) (layer "Edge.Cuts"))
 (gr_line (start 159 96) (end 126.25 96) (stroke (width 0.05) (type default)) (layer "Edge.Cuts"))
 (segment (start 135.95 103.75) (end 136 103.8) (width 0.15) (layer "F.Cu") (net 7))
 (segment (start 136.376 102.902834) (end 136.376 103.424) (width 0.15) (layer "F.Cu") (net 7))
 (segment (start 135.702834 102.624) (end 136.097166 102.624) (width 0.15) (layer "F.Cu") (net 7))
 (segment (start 134.245 102.75) (end 135.576834 102.75) (width 0.15) (layer "F.Cu") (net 7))
 (segment (start 135.576834 102.75) (end 135.702834 102.624) (width 0.15) (layer "F.Cu") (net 7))
 (segment (start 134.245 103.75) (end 135.95 103.75) (width 0.15) (layer "F.Cu") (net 7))
 (segment (start 136.097166 102.624) (end 136.376 102.902834) (width 0.15) (layer "F.Cu") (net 7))
 (segment (start 136.376 103.424) (end 136 103.8) (width 0.15) (layer "F.Cu") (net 7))
 (via (at 136 103.8) (size 0.4) (drill 0.2) (layers "F.Cu" "B.Cu") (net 7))
 (segment (start 140.482194 103.1) (end 141.4675 103.1) (width 0.15) (layer "B.Cu") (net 7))
 (segment (start 136 103.8) (end 136.736 103.064) (width 0.15) (layer "B.Cu") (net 7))
 (segment (start 136.736 103.064) (end 140.446194 103.064) (width 0.15) (layer "B.Cu") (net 7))
 (segment (start 140.446194 103.064) (end 140.482194 103.1) (width 0.15) (layer "B.Cu") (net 7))
 (segment (start 132.95 104.25) (end 134.245 104.25) (width 0.15) (layer "F.Cu") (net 6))
 (segment (start 134.245 103.25) (end 133.05 103.25) (width 0.15) (layer "F.Cu") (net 6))
 (segment (start 135.75 103.25) (end 135.9 103.1) (width 0.15) (layer "F.Cu") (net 6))
 (segment (start 132.8 104.1) (end 132.95 104.25) (width 0.15) (layer "F.Cu") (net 6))
 (segment (start 133.05 103.25) (end 132.8 103.5) (width 0.15) (layer "F.Cu") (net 6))
 (segment (start 134.245 103.25) (end 135.75 103.25) (width 0.15) (layer "F.Cu") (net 6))
 (segment (start 132.8 103.5) (end 132.8 104.1) (width 0.15) (layer "F.Cu") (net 6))
 (via (at 135.9 103.1) (size 0.4) (drill 0.2) (layers "F.Cu" "B.Cu") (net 6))
 (segment (start 136.3 102.7) (end 141.4675 102.7) (width 0.15) (layer "B.Cu") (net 6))
 (segment (start 135.9 103.1) (end 136.3 102.7) (width 0.15) (layer "B.Cu") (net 6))
 (segment (start 136.4 102) (end 136.4 101.31) (width 0.15) (layer "F.Cu") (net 5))
 (segment (start 134.245 102.25) (end 136.15 102.25) (width 0.15) (layer "F.Cu") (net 5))
 (segment (start 136.15 102.25) (end 136.4 102) (width 0.15) (layer "F.Cu") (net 5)))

